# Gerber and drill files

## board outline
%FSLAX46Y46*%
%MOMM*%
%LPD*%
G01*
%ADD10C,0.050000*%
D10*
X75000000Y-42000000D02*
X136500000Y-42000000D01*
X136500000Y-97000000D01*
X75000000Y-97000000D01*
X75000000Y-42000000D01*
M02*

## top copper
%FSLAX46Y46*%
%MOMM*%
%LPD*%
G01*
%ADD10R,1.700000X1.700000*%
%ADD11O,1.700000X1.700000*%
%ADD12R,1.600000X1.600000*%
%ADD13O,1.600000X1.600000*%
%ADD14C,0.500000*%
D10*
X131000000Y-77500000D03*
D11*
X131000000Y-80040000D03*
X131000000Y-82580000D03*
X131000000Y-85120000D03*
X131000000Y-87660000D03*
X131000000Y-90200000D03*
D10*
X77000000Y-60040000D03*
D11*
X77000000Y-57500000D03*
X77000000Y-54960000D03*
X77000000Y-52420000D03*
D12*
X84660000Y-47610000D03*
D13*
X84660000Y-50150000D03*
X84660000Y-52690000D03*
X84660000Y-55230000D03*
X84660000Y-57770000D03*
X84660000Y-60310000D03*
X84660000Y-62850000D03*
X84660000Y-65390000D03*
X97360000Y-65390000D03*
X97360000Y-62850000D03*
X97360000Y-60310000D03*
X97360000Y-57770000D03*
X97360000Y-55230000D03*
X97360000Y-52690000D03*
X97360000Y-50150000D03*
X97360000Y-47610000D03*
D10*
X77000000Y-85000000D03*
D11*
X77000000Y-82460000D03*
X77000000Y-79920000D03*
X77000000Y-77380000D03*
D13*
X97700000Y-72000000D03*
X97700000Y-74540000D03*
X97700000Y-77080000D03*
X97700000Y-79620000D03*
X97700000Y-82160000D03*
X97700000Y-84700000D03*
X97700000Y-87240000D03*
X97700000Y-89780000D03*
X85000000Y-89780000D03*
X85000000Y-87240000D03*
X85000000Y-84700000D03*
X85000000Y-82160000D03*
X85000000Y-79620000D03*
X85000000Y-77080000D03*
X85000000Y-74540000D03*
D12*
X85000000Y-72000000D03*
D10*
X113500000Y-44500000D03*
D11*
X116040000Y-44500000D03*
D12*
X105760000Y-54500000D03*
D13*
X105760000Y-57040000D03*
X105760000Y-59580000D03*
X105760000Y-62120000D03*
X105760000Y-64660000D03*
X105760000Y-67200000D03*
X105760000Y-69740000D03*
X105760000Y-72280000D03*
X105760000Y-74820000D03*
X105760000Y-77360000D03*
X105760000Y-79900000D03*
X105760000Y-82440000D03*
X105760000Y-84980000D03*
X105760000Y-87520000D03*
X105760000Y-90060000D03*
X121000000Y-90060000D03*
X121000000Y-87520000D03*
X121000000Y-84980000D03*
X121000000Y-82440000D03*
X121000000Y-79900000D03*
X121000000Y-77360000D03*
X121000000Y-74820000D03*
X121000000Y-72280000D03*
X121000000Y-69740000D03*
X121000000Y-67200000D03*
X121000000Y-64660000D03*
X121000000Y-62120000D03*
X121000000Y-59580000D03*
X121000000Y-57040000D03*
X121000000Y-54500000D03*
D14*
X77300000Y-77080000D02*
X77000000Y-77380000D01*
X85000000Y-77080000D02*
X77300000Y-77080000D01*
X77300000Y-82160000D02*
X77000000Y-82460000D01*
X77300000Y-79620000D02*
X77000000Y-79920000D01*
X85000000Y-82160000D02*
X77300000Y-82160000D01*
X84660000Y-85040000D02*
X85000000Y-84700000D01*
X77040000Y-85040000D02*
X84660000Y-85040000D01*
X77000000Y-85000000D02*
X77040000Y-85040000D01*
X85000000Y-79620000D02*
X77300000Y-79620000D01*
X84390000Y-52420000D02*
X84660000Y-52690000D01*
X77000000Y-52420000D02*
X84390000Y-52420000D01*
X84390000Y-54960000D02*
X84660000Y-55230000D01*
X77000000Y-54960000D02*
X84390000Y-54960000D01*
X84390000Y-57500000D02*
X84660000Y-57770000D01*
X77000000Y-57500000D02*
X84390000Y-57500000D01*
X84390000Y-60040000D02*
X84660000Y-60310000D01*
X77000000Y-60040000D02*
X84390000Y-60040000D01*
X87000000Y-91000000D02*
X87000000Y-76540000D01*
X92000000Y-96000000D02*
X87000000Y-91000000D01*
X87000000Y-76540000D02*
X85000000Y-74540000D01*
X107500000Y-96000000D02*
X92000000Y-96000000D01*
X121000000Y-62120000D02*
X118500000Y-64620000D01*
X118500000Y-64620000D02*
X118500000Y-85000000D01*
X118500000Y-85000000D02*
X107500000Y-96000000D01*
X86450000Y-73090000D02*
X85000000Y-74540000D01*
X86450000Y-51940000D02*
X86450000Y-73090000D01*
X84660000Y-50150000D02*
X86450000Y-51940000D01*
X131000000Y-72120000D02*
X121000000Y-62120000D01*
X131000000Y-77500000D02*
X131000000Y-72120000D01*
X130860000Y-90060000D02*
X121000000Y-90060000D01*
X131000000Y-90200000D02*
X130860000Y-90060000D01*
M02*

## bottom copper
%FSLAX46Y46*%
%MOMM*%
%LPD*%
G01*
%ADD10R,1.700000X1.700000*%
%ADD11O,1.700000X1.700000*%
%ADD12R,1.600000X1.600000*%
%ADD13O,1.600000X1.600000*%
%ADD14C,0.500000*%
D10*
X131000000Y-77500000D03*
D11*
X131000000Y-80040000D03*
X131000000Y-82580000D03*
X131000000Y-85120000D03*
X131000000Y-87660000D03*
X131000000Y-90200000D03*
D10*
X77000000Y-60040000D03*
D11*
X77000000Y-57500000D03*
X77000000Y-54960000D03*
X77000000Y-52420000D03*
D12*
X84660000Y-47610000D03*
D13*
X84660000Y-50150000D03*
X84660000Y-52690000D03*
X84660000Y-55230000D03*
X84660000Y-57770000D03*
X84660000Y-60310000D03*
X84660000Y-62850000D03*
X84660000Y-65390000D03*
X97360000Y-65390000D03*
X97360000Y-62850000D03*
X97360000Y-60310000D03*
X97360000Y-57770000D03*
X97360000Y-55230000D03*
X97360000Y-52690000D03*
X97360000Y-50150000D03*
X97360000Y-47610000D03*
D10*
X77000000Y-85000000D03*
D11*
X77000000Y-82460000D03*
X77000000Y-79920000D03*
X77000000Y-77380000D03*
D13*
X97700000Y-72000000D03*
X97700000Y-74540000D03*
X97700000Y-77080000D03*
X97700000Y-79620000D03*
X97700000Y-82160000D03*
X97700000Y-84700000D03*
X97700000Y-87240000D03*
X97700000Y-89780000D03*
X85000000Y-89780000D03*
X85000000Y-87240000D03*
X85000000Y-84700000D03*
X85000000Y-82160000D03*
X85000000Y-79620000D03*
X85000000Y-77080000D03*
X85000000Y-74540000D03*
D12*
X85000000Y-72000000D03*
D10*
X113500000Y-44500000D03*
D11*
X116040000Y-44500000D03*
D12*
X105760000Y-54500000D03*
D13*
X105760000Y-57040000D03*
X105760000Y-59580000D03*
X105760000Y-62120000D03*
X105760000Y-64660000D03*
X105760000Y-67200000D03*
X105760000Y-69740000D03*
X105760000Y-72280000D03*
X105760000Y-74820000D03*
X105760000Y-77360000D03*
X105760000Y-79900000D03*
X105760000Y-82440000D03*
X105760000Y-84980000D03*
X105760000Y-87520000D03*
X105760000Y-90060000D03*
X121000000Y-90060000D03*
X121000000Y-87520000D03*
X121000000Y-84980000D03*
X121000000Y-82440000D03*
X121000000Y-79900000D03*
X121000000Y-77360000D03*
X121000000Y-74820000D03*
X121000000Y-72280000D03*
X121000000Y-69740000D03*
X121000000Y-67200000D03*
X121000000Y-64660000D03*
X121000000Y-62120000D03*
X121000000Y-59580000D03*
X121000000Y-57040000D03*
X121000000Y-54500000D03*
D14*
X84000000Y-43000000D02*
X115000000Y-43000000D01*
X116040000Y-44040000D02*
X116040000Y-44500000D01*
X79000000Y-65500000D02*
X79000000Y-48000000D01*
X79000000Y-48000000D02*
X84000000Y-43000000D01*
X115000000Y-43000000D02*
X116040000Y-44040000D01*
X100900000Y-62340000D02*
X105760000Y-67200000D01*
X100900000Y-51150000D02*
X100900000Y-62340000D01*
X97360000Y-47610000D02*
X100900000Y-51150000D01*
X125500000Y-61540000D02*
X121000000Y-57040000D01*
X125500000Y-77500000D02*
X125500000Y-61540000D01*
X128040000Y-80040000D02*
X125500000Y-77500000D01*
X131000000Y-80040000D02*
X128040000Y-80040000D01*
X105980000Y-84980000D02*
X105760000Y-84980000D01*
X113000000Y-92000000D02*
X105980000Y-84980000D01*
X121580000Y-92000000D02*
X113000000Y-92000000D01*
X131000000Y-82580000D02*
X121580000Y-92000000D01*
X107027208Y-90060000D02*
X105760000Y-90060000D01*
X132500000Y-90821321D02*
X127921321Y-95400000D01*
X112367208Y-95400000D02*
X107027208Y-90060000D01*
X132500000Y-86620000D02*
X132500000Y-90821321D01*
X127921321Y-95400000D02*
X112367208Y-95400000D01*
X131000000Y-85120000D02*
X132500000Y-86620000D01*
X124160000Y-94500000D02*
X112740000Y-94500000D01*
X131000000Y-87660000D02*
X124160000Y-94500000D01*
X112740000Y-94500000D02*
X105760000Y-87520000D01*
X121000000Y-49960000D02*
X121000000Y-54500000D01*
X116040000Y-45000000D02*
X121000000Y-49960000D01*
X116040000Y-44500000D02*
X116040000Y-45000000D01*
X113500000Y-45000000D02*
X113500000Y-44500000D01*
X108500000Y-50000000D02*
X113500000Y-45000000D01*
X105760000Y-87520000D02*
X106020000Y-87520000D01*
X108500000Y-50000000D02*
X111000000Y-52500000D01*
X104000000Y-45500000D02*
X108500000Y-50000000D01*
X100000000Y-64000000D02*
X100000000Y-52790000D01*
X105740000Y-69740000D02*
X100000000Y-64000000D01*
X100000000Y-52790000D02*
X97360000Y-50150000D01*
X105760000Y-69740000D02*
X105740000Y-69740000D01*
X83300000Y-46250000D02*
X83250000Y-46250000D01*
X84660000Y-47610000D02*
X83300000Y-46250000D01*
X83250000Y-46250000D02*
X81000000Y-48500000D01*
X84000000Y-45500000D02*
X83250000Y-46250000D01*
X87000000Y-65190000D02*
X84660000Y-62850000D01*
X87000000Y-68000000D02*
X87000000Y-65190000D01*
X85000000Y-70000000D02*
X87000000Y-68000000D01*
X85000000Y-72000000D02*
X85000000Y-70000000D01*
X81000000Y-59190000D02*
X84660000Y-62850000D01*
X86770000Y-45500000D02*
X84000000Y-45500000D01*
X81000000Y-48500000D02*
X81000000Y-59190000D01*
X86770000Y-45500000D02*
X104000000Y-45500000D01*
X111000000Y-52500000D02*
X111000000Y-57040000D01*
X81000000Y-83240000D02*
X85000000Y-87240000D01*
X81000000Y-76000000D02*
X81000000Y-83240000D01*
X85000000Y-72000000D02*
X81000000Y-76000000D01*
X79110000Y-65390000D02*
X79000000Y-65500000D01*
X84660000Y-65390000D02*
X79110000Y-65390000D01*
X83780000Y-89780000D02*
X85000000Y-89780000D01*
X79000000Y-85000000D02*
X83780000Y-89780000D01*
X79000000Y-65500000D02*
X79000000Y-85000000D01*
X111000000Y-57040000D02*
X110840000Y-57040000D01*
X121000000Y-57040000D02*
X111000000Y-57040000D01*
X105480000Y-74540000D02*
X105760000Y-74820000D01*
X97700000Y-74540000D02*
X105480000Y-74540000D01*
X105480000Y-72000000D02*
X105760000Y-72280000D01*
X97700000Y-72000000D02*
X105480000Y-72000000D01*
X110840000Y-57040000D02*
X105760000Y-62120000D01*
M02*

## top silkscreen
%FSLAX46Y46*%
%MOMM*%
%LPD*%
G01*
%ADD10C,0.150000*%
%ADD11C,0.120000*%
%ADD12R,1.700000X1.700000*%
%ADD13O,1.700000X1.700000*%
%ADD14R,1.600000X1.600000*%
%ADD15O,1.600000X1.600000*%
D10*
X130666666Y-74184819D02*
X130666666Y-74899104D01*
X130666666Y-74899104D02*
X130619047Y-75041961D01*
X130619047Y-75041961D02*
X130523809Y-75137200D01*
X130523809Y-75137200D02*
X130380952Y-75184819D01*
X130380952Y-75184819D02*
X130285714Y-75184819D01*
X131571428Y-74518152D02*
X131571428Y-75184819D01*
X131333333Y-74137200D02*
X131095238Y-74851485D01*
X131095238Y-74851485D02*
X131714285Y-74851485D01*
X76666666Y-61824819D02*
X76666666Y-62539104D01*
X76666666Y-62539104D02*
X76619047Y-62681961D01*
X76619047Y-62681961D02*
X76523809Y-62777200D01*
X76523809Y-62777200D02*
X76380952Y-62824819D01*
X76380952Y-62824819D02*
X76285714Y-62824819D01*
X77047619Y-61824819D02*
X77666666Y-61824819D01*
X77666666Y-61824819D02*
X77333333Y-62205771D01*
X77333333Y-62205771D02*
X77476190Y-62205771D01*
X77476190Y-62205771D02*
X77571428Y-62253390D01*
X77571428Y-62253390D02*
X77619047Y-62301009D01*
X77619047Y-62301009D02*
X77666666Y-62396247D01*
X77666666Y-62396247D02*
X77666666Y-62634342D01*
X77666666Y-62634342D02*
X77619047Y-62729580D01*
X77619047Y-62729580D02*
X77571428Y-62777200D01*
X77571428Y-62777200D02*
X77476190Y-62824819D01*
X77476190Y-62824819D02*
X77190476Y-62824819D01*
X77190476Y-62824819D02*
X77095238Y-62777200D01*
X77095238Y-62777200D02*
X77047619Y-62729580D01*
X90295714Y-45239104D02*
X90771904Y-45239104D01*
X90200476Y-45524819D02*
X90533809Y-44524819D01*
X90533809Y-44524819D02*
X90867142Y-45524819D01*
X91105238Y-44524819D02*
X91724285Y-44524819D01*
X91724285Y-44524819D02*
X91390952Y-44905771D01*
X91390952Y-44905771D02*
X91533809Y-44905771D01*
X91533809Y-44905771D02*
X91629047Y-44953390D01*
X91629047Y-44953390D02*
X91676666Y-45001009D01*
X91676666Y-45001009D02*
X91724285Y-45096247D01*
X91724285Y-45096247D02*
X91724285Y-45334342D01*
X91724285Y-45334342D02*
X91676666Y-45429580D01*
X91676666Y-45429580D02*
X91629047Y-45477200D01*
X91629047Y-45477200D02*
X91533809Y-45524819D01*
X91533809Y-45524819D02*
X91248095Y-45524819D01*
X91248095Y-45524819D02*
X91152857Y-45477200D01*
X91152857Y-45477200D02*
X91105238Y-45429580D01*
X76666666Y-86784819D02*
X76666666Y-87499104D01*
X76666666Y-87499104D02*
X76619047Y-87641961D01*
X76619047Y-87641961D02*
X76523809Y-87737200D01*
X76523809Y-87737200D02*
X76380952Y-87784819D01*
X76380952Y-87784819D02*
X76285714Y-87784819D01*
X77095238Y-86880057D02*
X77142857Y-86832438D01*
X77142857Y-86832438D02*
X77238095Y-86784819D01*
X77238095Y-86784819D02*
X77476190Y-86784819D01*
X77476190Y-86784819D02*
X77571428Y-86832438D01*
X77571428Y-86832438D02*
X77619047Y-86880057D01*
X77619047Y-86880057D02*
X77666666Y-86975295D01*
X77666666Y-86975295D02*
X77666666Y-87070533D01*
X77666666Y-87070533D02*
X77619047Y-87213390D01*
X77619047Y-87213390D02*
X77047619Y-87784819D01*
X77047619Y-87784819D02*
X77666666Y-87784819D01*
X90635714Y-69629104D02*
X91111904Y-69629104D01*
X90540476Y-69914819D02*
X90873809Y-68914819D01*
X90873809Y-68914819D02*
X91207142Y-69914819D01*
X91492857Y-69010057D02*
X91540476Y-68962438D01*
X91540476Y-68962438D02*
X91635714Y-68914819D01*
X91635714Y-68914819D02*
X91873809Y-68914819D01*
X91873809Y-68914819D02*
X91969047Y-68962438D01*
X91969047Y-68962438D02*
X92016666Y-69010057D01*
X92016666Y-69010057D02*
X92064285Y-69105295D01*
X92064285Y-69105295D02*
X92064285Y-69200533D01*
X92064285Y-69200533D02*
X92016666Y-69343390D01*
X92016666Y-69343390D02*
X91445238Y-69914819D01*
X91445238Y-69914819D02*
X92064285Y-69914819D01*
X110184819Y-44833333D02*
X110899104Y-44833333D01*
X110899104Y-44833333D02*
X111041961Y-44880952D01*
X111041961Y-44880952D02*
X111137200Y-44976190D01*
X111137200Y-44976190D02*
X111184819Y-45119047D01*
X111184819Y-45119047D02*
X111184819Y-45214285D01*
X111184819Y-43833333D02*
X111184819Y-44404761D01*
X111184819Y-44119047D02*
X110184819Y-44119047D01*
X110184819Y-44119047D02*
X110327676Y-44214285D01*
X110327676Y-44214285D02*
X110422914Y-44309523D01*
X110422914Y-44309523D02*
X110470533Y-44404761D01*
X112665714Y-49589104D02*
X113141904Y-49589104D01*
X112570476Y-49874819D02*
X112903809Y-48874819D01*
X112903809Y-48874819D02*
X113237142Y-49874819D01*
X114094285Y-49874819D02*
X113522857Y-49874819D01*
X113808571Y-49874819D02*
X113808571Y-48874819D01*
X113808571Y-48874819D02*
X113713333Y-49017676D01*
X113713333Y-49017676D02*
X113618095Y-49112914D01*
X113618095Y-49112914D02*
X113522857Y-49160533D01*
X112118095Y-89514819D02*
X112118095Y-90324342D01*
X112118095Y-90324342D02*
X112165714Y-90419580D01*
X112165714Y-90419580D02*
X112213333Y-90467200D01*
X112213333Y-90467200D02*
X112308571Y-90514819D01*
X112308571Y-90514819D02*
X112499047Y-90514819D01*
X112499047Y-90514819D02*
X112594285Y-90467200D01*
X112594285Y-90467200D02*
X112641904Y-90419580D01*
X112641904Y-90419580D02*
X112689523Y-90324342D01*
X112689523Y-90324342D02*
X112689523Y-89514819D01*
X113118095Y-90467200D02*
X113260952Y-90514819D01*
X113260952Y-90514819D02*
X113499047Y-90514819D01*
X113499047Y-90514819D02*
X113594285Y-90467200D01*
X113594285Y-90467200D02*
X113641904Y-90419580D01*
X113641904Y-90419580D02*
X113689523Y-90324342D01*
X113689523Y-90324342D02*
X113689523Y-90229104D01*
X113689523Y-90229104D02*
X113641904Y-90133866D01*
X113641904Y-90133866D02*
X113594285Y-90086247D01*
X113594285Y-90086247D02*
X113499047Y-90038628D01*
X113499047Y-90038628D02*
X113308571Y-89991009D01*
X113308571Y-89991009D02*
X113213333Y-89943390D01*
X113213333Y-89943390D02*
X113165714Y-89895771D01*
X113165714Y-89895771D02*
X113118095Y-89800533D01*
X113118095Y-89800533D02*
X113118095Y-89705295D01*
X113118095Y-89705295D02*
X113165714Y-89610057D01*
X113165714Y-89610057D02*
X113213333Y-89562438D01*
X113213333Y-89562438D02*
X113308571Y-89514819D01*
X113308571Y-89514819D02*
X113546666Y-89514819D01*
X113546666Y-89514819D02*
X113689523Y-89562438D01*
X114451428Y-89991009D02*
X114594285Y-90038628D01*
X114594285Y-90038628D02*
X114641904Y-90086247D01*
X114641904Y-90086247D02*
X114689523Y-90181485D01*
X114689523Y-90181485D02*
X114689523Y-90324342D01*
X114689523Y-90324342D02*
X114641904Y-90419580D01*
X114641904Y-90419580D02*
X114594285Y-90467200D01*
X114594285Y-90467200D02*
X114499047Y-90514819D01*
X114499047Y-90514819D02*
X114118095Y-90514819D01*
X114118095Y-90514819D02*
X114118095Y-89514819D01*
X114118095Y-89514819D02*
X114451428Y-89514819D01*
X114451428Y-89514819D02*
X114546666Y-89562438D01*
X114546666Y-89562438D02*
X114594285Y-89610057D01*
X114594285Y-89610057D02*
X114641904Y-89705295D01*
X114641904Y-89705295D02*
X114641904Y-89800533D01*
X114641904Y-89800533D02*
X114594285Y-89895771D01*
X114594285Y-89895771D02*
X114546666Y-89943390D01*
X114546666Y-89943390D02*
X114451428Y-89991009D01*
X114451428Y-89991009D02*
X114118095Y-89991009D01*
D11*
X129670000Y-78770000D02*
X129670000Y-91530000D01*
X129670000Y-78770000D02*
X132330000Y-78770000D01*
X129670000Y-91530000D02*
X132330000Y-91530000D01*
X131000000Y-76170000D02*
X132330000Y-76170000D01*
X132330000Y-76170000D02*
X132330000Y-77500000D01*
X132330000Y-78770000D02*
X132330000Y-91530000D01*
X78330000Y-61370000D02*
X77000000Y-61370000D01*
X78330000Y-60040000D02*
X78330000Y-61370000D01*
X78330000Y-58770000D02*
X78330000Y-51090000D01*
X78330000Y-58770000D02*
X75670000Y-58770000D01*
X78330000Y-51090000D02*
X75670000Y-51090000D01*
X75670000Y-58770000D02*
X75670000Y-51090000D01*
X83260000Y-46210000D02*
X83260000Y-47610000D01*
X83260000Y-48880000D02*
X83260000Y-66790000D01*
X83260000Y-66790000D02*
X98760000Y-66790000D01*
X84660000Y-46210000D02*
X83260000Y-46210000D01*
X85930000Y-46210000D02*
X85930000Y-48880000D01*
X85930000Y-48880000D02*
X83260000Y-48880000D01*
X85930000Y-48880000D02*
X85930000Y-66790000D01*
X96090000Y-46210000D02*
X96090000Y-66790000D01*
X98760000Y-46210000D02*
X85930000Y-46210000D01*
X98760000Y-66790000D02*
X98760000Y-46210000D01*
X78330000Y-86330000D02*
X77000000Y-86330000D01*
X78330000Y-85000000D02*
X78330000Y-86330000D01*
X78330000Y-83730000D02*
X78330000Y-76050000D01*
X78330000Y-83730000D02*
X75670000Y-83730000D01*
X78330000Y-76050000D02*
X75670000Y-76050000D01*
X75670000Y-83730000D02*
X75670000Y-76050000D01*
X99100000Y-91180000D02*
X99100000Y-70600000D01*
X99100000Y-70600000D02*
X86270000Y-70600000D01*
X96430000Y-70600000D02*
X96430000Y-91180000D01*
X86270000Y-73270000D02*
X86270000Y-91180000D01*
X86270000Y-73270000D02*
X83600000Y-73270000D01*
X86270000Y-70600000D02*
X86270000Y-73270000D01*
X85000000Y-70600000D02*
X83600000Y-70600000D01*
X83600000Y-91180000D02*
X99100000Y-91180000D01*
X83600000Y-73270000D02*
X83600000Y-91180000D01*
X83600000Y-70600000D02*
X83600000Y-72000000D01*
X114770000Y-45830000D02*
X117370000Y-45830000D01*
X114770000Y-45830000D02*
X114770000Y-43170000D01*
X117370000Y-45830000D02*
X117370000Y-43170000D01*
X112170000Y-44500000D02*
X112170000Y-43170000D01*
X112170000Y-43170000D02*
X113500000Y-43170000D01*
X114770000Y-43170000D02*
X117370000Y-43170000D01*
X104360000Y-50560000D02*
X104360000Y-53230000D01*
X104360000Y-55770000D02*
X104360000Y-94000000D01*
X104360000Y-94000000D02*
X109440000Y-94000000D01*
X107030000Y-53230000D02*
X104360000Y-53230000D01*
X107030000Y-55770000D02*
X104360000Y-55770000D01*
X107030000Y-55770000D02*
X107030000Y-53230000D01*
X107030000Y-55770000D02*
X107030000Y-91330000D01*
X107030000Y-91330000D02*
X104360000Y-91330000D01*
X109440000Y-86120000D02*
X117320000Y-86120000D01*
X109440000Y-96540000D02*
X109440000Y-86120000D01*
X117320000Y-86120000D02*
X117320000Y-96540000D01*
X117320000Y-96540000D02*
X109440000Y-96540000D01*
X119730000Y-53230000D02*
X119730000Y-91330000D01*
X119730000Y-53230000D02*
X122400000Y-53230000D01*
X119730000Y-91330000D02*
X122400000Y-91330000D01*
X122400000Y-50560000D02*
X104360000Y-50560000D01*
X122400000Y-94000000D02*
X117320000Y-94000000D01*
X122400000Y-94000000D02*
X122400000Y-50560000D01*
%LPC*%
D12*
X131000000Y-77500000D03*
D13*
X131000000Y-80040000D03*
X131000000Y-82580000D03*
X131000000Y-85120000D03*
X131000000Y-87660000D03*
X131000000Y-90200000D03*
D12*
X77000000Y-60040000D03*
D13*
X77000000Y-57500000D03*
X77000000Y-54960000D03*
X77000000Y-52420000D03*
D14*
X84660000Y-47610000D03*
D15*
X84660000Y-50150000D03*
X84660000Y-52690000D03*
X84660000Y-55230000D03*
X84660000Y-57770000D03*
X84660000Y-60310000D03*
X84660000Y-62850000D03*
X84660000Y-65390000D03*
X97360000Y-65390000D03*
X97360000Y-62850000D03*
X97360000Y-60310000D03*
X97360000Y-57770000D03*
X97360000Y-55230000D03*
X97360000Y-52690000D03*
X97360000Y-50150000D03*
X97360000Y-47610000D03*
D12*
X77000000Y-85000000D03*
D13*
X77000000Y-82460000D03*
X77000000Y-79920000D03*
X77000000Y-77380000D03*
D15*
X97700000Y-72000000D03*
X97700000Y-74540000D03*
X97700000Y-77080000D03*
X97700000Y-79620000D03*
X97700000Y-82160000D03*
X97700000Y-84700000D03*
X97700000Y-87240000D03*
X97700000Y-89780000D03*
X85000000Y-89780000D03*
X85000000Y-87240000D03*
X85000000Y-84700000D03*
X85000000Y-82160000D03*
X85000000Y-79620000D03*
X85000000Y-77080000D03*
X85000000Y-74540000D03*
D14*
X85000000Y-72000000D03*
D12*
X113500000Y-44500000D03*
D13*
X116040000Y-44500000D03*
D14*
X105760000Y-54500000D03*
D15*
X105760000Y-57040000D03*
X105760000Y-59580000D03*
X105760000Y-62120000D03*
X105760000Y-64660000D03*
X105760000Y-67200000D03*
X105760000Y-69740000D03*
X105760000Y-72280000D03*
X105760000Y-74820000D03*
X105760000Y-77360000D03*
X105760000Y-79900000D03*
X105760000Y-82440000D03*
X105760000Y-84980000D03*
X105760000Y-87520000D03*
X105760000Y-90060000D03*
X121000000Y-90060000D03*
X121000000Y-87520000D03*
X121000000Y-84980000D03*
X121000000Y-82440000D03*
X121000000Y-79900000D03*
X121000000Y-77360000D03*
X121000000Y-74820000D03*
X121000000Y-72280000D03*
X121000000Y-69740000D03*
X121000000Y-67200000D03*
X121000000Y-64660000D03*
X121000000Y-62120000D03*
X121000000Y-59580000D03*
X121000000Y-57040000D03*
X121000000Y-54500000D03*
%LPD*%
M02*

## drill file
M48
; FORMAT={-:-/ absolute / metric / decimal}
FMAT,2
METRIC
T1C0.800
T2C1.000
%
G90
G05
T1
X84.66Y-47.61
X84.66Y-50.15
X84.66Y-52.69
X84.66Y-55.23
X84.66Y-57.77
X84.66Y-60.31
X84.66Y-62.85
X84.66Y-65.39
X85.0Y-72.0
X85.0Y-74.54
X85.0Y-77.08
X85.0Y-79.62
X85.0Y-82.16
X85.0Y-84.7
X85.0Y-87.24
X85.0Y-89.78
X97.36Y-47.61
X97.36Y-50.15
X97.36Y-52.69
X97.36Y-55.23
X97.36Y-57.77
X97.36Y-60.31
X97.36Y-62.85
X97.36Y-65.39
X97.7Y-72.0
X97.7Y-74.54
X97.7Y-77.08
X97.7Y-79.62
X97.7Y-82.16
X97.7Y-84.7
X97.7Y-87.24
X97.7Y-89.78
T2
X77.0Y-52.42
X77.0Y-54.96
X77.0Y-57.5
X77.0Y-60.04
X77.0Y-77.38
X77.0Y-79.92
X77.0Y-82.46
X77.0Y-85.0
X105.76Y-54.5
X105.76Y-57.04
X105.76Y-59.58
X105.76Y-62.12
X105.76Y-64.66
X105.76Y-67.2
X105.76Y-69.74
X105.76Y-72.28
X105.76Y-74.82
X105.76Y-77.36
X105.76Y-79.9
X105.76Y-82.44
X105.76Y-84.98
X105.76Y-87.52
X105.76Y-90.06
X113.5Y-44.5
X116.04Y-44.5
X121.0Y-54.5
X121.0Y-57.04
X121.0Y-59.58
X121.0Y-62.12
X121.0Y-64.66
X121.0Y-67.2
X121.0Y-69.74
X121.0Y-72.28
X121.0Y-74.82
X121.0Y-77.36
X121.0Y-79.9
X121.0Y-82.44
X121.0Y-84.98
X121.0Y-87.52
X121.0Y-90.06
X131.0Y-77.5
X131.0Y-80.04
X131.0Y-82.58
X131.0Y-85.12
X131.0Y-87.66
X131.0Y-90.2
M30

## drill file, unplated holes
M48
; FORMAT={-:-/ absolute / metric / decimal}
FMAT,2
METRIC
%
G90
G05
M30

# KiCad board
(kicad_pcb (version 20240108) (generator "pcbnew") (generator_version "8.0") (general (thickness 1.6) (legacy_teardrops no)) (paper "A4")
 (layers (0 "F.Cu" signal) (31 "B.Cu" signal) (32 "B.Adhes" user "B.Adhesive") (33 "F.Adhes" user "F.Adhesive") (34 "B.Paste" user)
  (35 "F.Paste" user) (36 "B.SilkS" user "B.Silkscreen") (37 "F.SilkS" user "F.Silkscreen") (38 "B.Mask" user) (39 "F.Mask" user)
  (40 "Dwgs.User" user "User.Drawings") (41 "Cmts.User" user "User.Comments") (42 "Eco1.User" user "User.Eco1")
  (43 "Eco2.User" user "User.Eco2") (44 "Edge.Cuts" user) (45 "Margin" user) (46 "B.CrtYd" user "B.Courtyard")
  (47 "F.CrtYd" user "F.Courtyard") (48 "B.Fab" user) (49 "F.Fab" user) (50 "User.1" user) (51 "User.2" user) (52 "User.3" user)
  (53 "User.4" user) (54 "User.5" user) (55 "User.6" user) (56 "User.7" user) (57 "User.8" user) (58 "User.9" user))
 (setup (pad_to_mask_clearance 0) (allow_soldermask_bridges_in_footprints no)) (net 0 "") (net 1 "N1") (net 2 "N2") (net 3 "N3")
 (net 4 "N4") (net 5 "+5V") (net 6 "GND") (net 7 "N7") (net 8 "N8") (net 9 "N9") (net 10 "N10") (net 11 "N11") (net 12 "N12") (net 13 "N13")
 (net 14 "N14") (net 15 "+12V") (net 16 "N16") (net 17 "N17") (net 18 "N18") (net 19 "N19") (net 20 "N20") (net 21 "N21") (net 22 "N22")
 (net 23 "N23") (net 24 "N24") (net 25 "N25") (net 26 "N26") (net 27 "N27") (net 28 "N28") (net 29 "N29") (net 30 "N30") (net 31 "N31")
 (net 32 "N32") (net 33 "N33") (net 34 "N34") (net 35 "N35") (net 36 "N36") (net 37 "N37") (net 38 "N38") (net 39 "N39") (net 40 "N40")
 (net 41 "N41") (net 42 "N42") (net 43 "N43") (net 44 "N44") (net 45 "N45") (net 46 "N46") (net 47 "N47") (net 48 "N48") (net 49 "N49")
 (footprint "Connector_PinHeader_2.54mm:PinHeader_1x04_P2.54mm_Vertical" (layer "F.Cu") (at 77 85 180)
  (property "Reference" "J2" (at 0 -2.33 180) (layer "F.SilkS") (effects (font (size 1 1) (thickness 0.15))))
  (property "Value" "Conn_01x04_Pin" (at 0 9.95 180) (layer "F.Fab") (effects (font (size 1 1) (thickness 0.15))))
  (fp_line (start 1.33 1.27) (end 1.33 8.95) (stroke (width 0.12) (type solid)) (layer "F.SilkS"))
  (fp_line (start -1.33 8.95) (end 1.33 8.95) (stroke (width 0.12) (type solid)) (layer "F.SilkS"))
  (fp_line (start -1.33 1.27) (end 1.33 1.27) (stroke (width 0.12) (type solid)) (layer "F.SilkS"))
  (fp_line (start -1.33 1.27) (end -1.33 8.95) (stroke (width 0.12) (type solid)) (layer "F.SilkS"))
  (fp_line (start -1.33 0) (end -1.33 -1.33) (stroke (width 0.12) (type solid)) (layer "F.SilkS"))
  (fp_line (start -1.33 -1.33) (end 0 -1.33) (stroke (width 0.12) (type solid)) (layer "F.SilkS"))
  (pad "1" thru_hole rect (at 0 0 180) (size 1.7 1.7) (drill 1) (layers "*.Cu" "*.Mask") (remove_unused_layers no) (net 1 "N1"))
  (pad "2" thru_hole oval (at 0 2.54 180) (size 1.7 1.7) (drill 1) (layers "*.Cu" "*.Mask") (remove_unused_layers no) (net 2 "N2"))
  (pad "3" thru_hole oval (at 0 5.08 180) (size 1.7 1.7) (drill 1) (layers "*.Cu" "*.Mask") (remove_unused_layers no) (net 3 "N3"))
  (pad "4" thru_hole oval (at 0 7.62 180) (size 1.7 1.7) (drill 1) (layers "*.Cu" "*.Mask") (remove_unused_layers no) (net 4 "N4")))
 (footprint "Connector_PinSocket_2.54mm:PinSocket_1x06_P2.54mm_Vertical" (layer "F.Cu") (at 131 77.5)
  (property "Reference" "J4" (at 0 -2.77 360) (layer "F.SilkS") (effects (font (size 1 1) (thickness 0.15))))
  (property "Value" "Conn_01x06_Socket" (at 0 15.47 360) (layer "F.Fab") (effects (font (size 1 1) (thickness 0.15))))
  (fp_line (start -1.33 1.27) (end -1.33 14.03) (stroke (width 0.12) (type solid)) (layer "F.SilkS"))
  (fp_line (start -1.33 1.27) (end 1.33 1.27) (stroke (width 0.12) (type solid)) (layer "F.SilkS"))
  (fp_line (start -1.33 14.03) (end 1.33 14.03) (stroke (width 0.12) (type solid)) (layer "F.SilkS"))
  (fp_line (start 0 -1.33) (end 1.33 -1.33) (stroke (width 0.12) (type solid)) (layer "F.SilkS"))
  (fp_line (start 1.33 -1.33) (end 1.33 0) (stroke (width 0.12) (type solid)) (layer "F.SilkS"))
  (fp_line (start 1.33 1.27) (end 1.33 14.03) (stroke (width 0.12) (type solid)) (layer "F.SilkS"))
  (pad "1" thru_hole rect (at 0 0) (size 1.7 1.7) (drill 1) (layers "*.Cu" "*.Mask") (remove_unused_layers no) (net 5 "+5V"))
  (pad "2" thru_hole oval (at 0 2.54) (size 1.7 1.7) (drill 1) (layers "*.Cu" "*.Mask") (remove_unused_layers no) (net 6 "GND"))
  (pad "3" thru_hole oval (at 0 5.08) (size 1.7 1.7) (drill 1) (layers "*.Cu" "*.Mask") (remove_unused_layers no) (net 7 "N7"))
  (pad "4" thru_hole oval (at 0 7.62) (size 1.7 1.7) (drill 1) (layers "*.Cu" "*.Mask") (remove_unused_layers no) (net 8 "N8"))
  (pad "5" thru_hole oval (at 0 10.16) (size 1.7 1.7) (drill 1) (layers "*.Cu" "*.Mask") (remove_unused_layers no) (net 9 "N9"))
  (pad "6" thru_hole oval (at 0 12.7) (size 1.7 1.7) (drill 1) (layers "*.Cu" "*.Mask") (remove_unused_layers no) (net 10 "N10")))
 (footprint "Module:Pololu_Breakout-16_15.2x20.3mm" (layer "F.Cu") (at 84.66 47.61)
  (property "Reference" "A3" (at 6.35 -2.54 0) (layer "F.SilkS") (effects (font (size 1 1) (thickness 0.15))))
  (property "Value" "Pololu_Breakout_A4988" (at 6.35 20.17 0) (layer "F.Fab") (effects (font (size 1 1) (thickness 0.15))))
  (fp_line (start -1.4 -1.4) (end -1.4 0) (stroke (width 0.12) (type solid)) (layer "F.SilkS"))
  (fp_line (start -1.4 1.27) (end -1.4 19.18) (stroke (width 0.12) (type solid)) (layer "F.SilkS"))
  (fp_line (start -1.4 19.18) (end 14.1 19.18) (stroke (width 0.12) (type solid)) (layer "F.SilkS"))
  (fp_line (start 0 -1.4) (end -1.4 -1.4) (stroke (width 0.12) (type solid)) (layer "F.SilkS"))
  (fp_line (start 1.27 -1.4) (end 1.27 1.27) (stroke (width 0.12) (type solid)) (layer "F.SilkS"))
  (fp_line (start 1.27 1.27) (end -1.4 1.27) (stroke (width 0.12) (type solid)) (layer "F.SilkS"))
  (fp_line (start 1.27 1.27) (end 1.27 19.18) (stroke (width 0.12) (type solid)) (layer "F.SilkS"))
  (fp_line (start 11.43 -1.4) (end 11.43 19.18) (stroke (width 0.12) (type solid)) (layer "F.SilkS"))
  (fp_line (start 14.1 -1.4) (end 1.27 -1.4) (stroke (width 0.12) (type solid)) (layer "F.SilkS"))
  (fp_line (start 14.1 19.18) (end 14.1 -1.4) (stroke (width 0.12) (type solid)) (layer "F.SilkS"))
  (pad "1" thru_hole rect (at 0 0) (size 1.6 1.6) (drill 0.8) (layers "*.Cu" "*.Mask") (remove_unused_layers no) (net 6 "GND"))
  (pad "2" thru_hole oval (at 0 2.54) (size 1.6 1.6) (drill 0.8) (layers "*.Cu" "*.Mask") (remove_unused_layers no) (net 5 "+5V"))
  (pad "3" thru_hole oval (at 0 5.08) (size 1.6 1.6) (drill 0.8) (layers "*.Cu" "*.Mask") (remove_unused_layers no) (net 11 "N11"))
  (pad "4" thru_hole oval (at 0 7.62) (size 1.6 1.6) (drill 0.8) (layers "*.Cu" "*.Mask") (remove_unused_layers no) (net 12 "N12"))
  (pad "5" thru_hole oval (at 0 10.16) (size 1.6 1.6) (drill 0.8) (layers "*.Cu" "*.Mask") (remove_unused_layers no) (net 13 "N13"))
  (pad "6" thru_hole oval (at 0 12.7) (size 1.6 1.6) (drill 0.8) (layers "*.Cu" "*.Mask") (remove_unused_layers no) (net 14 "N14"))
  (pad "7" thru_hole oval (at 0 15.24) (size 1.6 1.6) (drill 0.8) (layers "*.Cu" "*.Mask") (remove_unused_layers no) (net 6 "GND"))
  (pad "8" thru_hole oval (at 0 17.78) (size 1.6 1.6) (drill 0.8) (layers "*.Cu" "*.Mask") (remove_unused_layers no) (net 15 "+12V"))
  (pad "9" thru_hole oval (at 12.7 17.78) (size 1.6 1.6) (drill 0.8) (layers "*.Cu" "*.Mask") (remove_unused_layers no) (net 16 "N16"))
  (pad "10" thru_hole oval (at 12.7 15.24) (size 1.6 1.6) (drill 0.8) (layers "*.Cu" "*.Mask") (remove_unused_layers no) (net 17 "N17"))
  (pad "11" thru_hole oval (at 12.7 12.7) (size 1.6 1.6) (drill 0.8) (layers "*.Cu" "*.Mask") (remove_unused_layers no) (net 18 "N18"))
  (pad "12" thru_hole oval (at 12.7 10.16) (size 1.6 1.6) (drill 0.8) (layers "*.Cu" "*.Mask") (remove_unused_layers no) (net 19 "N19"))
  (pad "13" thru_hole oval (at 12.7 7.62) (size 1.6 1.6) (drill 0.8) (layers "*.Cu" "*.Mask") (remove_unused_layers no) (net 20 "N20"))
  (pad "14" thru_hole oval (at 12.7 5.08) (size 1.6 1.6) (drill 0.8) (layers "*.Cu" "*.Mask") (remove_unused_layers no) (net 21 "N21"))
  (pad "15" thru_hole oval (at 12.7 2.54) (size 1.6 1.6) (drill 0.8) (layers "*.Cu" "*.Mask") (remove_unused_layers no) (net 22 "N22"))
  (pad "16" thru_hole oval (at 12.7 0) (size 1.6 1.6) (drill 0.8) (layers "*.Cu" "*.Mask") (remove_unused_layers no) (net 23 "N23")))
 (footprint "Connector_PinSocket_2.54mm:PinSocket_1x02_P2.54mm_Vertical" (layer "F.Cu") (at 113.5 44.5 90)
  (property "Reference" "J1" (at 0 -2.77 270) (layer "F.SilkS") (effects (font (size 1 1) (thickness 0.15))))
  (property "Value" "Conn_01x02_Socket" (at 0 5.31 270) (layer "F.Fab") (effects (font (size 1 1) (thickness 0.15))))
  (fp_line (start 1.33 -1.33) (end 1.33 0) (stroke (width 0.12) (type solid)) (layer "F.SilkS"))
  (fp_line (start 0 -1.33) (end 1.33 -1.33) (stroke (width 0.12) (type solid)) (layer "F.SilkS"))
  (fp_line (start 1.33 1.27) (end 1.33 3.87) (stroke (width 0.12) (type solid)) (layer "F.SilkS"))
  (fp_line (start -1.33 1.27) (end 1.33 1.27) (stroke (width 0.12) (type solid)) (layer "F.SilkS"))
  (fp_line (start -1.33 1.27) (end -1.33 3.87) (stroke (width 0.12) (type solid)) (layer "F.SilkS"))
  (fp_line (start -1.33 3.87) (end 1.33 3.87) (stroke (width 0.12) (type solid)) (layer "F.SilkS"))
  (pad "1" thru_hole rect (at 0 0 90) (size 1.7 1.7) (drill 1) (layers "*.Cu" "*.Mask") (remove_unused_layers no) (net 6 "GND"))
  (pad "2" thru_hole oval (at 0 2.54 90) (size 1.7 1.7) (drill 1) (layers "*.Cu" "*.Mask") (remove_unused_layers no) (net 15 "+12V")))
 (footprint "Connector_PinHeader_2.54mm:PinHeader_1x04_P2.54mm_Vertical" (layer "F.Cu") (at 77 60.04 180)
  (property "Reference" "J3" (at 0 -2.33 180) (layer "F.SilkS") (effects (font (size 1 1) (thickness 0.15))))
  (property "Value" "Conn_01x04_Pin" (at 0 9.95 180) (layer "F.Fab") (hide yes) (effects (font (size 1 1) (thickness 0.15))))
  (fp_line (start 1.33 1.27) (end 1.33 8.95) (stroke (width 0.12) (type solid)) (layer "F.SilkS"))
  (fp_line (start -1.33 8.95) (end 1.33 8.95) (stroke (width 0.12) (type solid)) (layer "F.SilkS"))
  (fp_line (start -1.33 1.27) (end 1.33 1.27) (stroke (width 0.12) (type solid)) (layer "F.SilkS"))
  (fp_line (start -1.33 1.27) (end -1.33 8.95) (stroke (width 0.12) (type solid)) (layer "F.SilkS"))
  (fp_line (start -1.33 0) (end -1.33 -1.33) (stroke (width 0.12) (type solid)) (layer "F.SilkS"))
  (fp_line (start -1.33 -1.33) (end 0 -1.33) (stroke (width 0.12) (type solid)) (layer "F.SilkS"))
  (pad "1" thru_hole rect (at 0 0 180) (size 1.7 1.7) (drill 1) (layers "*.Cu" "*.Mask") (remove_unused_layers no) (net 14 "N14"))
  (pad "2" thru_hole oval (at 0 2.54 180) (size 1.7 1.7) (drill 1) (layers "*.Cu" "*.Mask") (remove_unused_layers no) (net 13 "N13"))
  (pad "3" thru_hole oval (at 0 5.08 180) (size 1.7 1.7) (drill 1) (layers "*.Cu" "*.Mask") (remove_unused_layers no) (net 12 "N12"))
  (pad "4" thru_hole oval (at 0 7.62 180) (size 1.7 1.7) (drill 1) (layers "*.Cu" "*.Mask") (remove_unused_layers no) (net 11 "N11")))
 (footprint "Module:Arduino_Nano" (layer "F.Cu") (at 105.76 54.5)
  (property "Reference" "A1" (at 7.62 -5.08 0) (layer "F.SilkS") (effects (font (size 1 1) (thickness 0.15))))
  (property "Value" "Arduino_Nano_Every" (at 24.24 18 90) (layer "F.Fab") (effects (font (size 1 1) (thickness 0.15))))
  (fp_line (start -1.4 -3.94) (end -1.4 -1.27) (stroke (width 0.12) (type solid)) (layer "F.SilkS"))
  (fp_line (start -1.4 1.27) (end -1.4 39.5) (stroke (width 0.12) (type solid)) (layer "F.SilkS"))
  (fp_line (start -1.4 39.5) (end 3.68 39.5) (stroke (width 0.12) (type solid)) (layer "F.SilkS"))
  (fp_line (start 1.27 -1.27) (end -1.4 -1.27) (stroke (width 0.12) (type solid)) (layer "F.SilkS"))
  (fp_line (start 1.27 1.27) (end -1.4 1.27) (stroke (width 0.12) (type solid)) (layer "F.SilkS"))
  (fp_line (start 1.27 1.27) (end 1.27 -1.27) (stroke (width 0.12) (type solid)) (layer "F.SilkS"))
  (fp_line (start 1.27 1.27) (end 1.27 36.83) (stroke (width 0.12) (type solid)) (layer "F.SilkS"))
  (fp_line (start 1.27 36.83) (end -1.4 36.83) (stroke (width 0.12) (type solid)) (layer "F.SilkS"))
  (fp_line (start 3.68 31.62) (end 11.56 31.62) (stroke (width 0.12) (type solid)) (layer "F.SilkS"))
  (fp_line (start 3.68 42.04) (end 3.68 31.62) (stroke (width 0.12) (type solid)) (layer "F.SilkS"))
  (fp_line (start 11.56 31.62) (end 11.56 42.04) (stroke (width 0.12) (type solid)) (layer "F.SilkS"))
  (fp_line (start 11.56 42.04) (end 3.68 42.04) (stroke (width 0.12) (type solid)) (layer "F.SilkS"))
  (fp_line (start 13.97 -1.27) (end 13.97 36.83) (stroke (width 0.12) (type solid)) (layer "F.SilkS"))
  (fp_line (start 13.97 -1.27) (end 16.64 -1.27) (stroke (width 0.12) (type solid)) (layer "F.SilkS"))
  (fp_line (start 13.97 36.83) (end 16.64 36.83) (stroke (width 0.12) (type solid)) (layer "F.SilkS"))
  (fp_line (start 16.64 -3.94) (end -1.4 -3.94) (stroke (width 0.12) (type solid)) (layer "F.SilkS"))
  (fp_line (start 16.64 39.5) (end 11.56 39.5) (stroke (width 0.12) (type solid)) (layer "F.SilkS"))
  (fp_line (start 16.64 39.5) (end 16.64 -3.94) (stroke (width 0.12) (type solid)) (layer "F.SilkS"))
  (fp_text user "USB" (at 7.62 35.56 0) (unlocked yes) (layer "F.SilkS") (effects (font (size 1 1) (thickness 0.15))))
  (pad "1" thru_hole rect (at 0 0) (size 1.6 1.6) (drill 1) (layers "*.Cu" "*.Mask") (remove_unused_layers no) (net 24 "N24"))
  (pad "2" thru_hole oval (at 0 2.54) (size 1.6 1.6) (drill 1) (layers "*.Cu" "*.Mask") (remove_unused_layers no) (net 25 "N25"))
  (pad "3" thru_hole oval (at 0 5.08) (size 1.6 1.6) (drill 1) (layers "*.Cu" "*.Mask") (remove_unused_layers no) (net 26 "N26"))
  (pad "4" thru_hole oval (at 0 7.62) (size 1.6 1.6) (drill 1) (layers "*.Cu" "*.Mask") (remove_unused_layers no) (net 6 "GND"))
  (pad "5" thru_hole oval (at 0 10.16) (size 1.6 1.6) (drill 1) (layers "*.Cu" "*.Mask") (remove_unused_layers no) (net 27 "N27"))
  (pad "6" thru_hole oval (at 0 12.7) (size 1.6 1.6) (drill 1) (layers "*.Cu" "*.Mask") (remove_unused_layers no) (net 23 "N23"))
  (pad "7" thru_hole oval (at 0 15.24) (size 1.6 1.6) (drill 1) (layers "*.Cu" "*.Mask") (remove_unused_layers no) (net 22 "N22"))
  (pad "8" thru_hole oval (at 0 17.78) (size 1.6 1.6) (drill 1) (layers "*.Cu" "*.Mask") (remove_unused_layers no) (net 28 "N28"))
  (pad "9" thru_hole oval (at 0 20.32) (size 1.6 1.6) (drill 1) (layers "*.Cu" "*.Mask") (remove_unused_layers no) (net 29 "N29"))
  (pad "10" thru_hole oval (at 0 22.86) (size 1.6 1.6) (drill 1) (layers "*.Cu" "*.Mask") (remove_unused_layers no) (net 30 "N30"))
  (pad "11" thru_hole oval (at 0 25.4) (size 1.6 1.6) (drill 1) (layers "*.Cu" "*.Mask") (remove_unused_layers no) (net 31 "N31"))
  (pad "12" thru_hole oval (at 0 27.94) (size 1.6 1.6) (drill 1) (layers "*.Cu" "*.Mask") (remove_unused_layers no) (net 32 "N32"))
  (pad "13" thru_hole oval (at 0 30.48) (size 1.6 1.6) (drill 1) (layers "*.Cu" "*.Mask") (remove_unused_layers no) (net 7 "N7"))
  (pad "14" thru_hole oval (at 0 33.02) (size 1.6 1.6) (drill 1) (layers "*.Cu" "*.Mask") (remove_unused_layers no) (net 9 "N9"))
  (pad "15" thru_hole oval (at 0 35.56) (size 1.6 1.6) (drill 1) (layers "*.Cu" "*.Mask") (remove_unused_layers no) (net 8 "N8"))
  (pad "16" thru_hole oval (at 15.24 35.56) (size 1.6 1.6) (drill 1) (layers "*.Cu" "*.Mask") (remove_unused_layers no) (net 10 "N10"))
  (pad "17" thru_hole oval (at 15.24 33.02) (size 1.6 1.6) (drill 1) (layers "*.Cu" "*.Mask") (remove_unused_layers no) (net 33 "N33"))
  (pad "18" thru_hole oval (at 15.24 30.48) (size 1.6 1.6) (drill 1) (layers "*.Cu" "*.Mask") (remove_unused_layers no) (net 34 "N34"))
  (pad "19" thru_hole oval (at 15.24 27.94) (size 1.6 1.6) (drill 1) (layers "*.Cu" "*.Mask") (remove_unused_layers no) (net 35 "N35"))
  (pad "20" thru_hole oval (at 15.24 25.4) (size 1.6 1.6) (drill 1) (layers "*.Cu" "*.Mask") (remove_unused_layers no) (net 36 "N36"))
  (pad "21" thru_hole oval (at 15.24 22.86) (size 1.6 1.6) (drill 1) (layers "*.Cu" "*.Mask") (remove_unused_layers no) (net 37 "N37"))
  (pad "22" thru_hole oval (at 15.24 20.32) (size 1.6 1.6) (drill 1) (layers "*.Cu" "*.Mask") (remove_unused_layers no) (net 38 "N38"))
  (pad "23" thru_hole oval (at 15.24 17.78) (size 1.6 1.6) (drill 1) (layers "*.Cu" "*.Mask") (remove_unused_layers no) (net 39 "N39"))
  (pad "24" thru_hole oval (at 15.24 15.24) (size 1.6 1.6) (drill 1) (layers "*.Cu" "*.Mask") (remove_unused_layers no) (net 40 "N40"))
  (pad "25" thru_hole oval (at 15.24 12.7) (size 1.6 1.6) (drill 1) (layers "*.Cu" "*.Mask") (remove_unused_layers no) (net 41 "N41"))
  (pad "26" thru_hole oval (at 15.24 10.16) (size 1.6 1.6) (drill 1) (layers "*.Cu" "*.Mask") (remove_unused_layers no) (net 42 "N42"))
  (pad "27" thru_hole oval (at 15.24 7.62) (size 1.6 1.6) (drill 1) (layers "*.Cu" "*.Mask") (remove_unused_layers no) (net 5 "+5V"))
  (pad "28" thru_hole oval (at 15.24 5.08) (size 1.6 1.6) (drill 1) (layers "*.Cu" "*.Mask") (remove_unused_layers no) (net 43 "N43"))
  (pad "29" thru_hole oval (at 15.24 2.54) (size 1.6 1.6) (drill 1) (layers "*.Cu" "*.Mask") (remove_unused_layers no) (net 6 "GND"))
  (pad "30" thru_hole oval (at 15.24 0) (size 1.6 1.6) (drill 1) (layers "*.Cu" "*.Mask") (remove_unused_layers no) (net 15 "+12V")))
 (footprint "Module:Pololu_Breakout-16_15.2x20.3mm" (layer "F.Cu") (at 85 72)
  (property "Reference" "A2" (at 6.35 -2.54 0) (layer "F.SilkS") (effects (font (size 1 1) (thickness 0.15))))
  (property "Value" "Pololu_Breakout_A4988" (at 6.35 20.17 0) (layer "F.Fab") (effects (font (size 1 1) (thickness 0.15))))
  (fp_line (start -1.4 -1.4) (end -1.4 0) (stroke (width 0.12) (type solid)) (layer "F.SilkS"))
  (fp_line (start -1.4 1.27) (end -1.4 19.18) (stroke (width 0.12) (type solid)) (layer "F.SilkS"))
  (fp_line (start -1.4 19.18) (end 14.1 19.18) (stroke (width 0.12) (type solid)) (layer "F.SilkS"))
  (fp_line (start 0 -1.4) (end -1.4 -1.4) (stroke (width 0.12) (type solid)) (layer "F.SilkS"))
  (fp_line (start 1.27 -1.4) (end 1.27 1.27) (stroke (width 0.12) (type solid)) (layer "F.SilkS"))
  (fp_line (start 1.27 1.27) (end -1.4 1.27) (stroke (width 0.12) (type solid)) (layer "F.SilkS"))
  (fp_line (start 1.27 1.27) (end 1.27 19.18) (stroke (width 0.12) (type solid)) (layer "F.SilkS"))
  (fp_line (start 11.43 -1.4) (end 11.43 19.18) (stroke (width 0.12) (type solid)) (layer "F.SilkS"))
  (fp_line (start 14.1 -1.4) (end 1.27 -1.4) (stroke (width 0.12) (type solid)) (layer "F.SilkS"))
  (fp_line (start 14.1 19.18) (end 14.1 -1.4) (stroke (width 0.12) (type solid)) (layer "F.SilkS"))
  (pad "1" thru_hole rect (at 0 0) (size 1.6 1.6) (drill 0.8) (layers "*.Cu" "*.Mask") (remove_unused_layers no) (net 6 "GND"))
  (pad "2" thru_hole oval (at 0 2.54) (size 1.6 1.6) (drill 0.8) (layers "*.Cu" "*.Mask") (remove_unused_layers no) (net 5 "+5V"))
  (pad "3" thru_hole oval (at 0 5.08) (size 1.6 1.6) (drill 0.8) (layers "*.Cu" "*.Mask") (remove_unused_layers no) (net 4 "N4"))
  (pad "4" thru_hole oval (at 0 7.62) (size 1.6 1.6) (drill 0.8) (layers "*.Cu" "*.Mask") (remove_unused_layers no) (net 3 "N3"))
  (pad "5" thru_hole oval (at 0 10.16) (size 1.6 1.6) (drill 0.8) (layers "*.Cu" "*.Mask") (remove_unused_layers no) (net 2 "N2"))
  (pad "6" thru_hole oval (at 0 12.7) (size 1.6 1.6) (drill 0.8) (layers "*.Cu" "*.Mask") (remove_unused_layers no) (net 1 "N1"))
  (pad "7" thru_hole oval (at 0 15.24) (size 1.6 1.6) (drill 0.8) (layers "*.Cu" "*.Mask") (remove_unused_layers no) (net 6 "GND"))
  (pad "8" thru_hole oval (at 0 17.78) (size 1.6 1.6) (drill 0.8) (layers "*.Cu" "*.Mask") (remove_unused_layers no) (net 15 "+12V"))
  (pad "9" thru_hole oval (at 12.7 17.78) (size 1.6 1.6) (drill 0.8) (layers "*.Cu" "*.Mask") (remove_unused_layers no) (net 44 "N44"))
  (pad "10" thru_hole oval (at 12.7 15.24) (size 1.6 1.6) (drill 0.8) (layers "*.Cu" "*.Mask") (remove_unused_layers no) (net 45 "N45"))
  (pad "11" thru_hole oval (at 12.7 12.7) (size 1.6 1.6) (drill 0.8) (layers "*.Cu" "*.Mask") (remove_unused_layers no) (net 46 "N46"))
  (pad "12" thru_hole oval (at 12.7 10.16) (size 1.6 1.6) (drill 0.8) (layers "*.Cu" "*.Mask") (remove_unused_layers no) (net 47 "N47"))
  (pad "13" thru_hole oval (at 12.7 7.62) (size 1.6 1.6) (drill 0.8) (layers "*.Cu" "*.Mask") (remove_unused_layers no) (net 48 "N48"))
  (pad "14" thru_hole oval (at 12.7 5.08) (size 1.6 1.6) (drill 0.8) (layers "*.Cu" "*.Mask") (remove_unused_layers no) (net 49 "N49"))
  (pad "15" thru_hole oval (at 12.7 2.54) (size 1.6 1.6) (drill 0.8) (layers "*.Cu" "*.Mask") (remove_unused_layers no) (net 29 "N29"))
  (pad "16" thru_hole oval (at 12.7 0) (size 1.6 1.6) (drill 0.8) (layers "*.Cu" "*.Mask") (remove_unused_layers no) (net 28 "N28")))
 (gr_rect (start 75 42) (end 136.5 97) (stroke (width 0.05) (type default)) (fill none) (layer "Edge.Cuts"))
 (segment (start 83.25 46.25) (end 81 48.5) (width 0.5) (layer "B.Cu") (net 6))
 (segment (start 81 76) (end 81 83.24) (width 0.5) (layer "B.Cu") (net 6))
 (segment (start 87 68) (end 87 65.19) (width 0.5) (layer "B.Cu") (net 6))
 (segment (start 104 45.5) (end 108.5 50) (width 0.5) (layer "B.Cu") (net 6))
 (segment (start 131 80.04) (end 128.04 80.04) (width 0.5) (layer "B.Cu") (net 6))
 (segment (start 81 48.5) (end 81 59.19) (width 0.5) (layer "B.Cu") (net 6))
 (segment (start 85 72) (end 85 70) (width 0.5) (layer "B.Cu") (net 6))
 (segment (start 86.77 45.5) (end 84 45.5) (width 0.5) (layer "B.Cu") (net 6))
 (segment (start 81 83.24) (end 85 87.24) (width 0.5) (layer "B.Cu") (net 6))
 (segment (start 125.5 77.5) (end 125.5 61.54) (width 0.5) (layer "B.Cu") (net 6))
 (segment (start 121 57.04) (end 111 57.04) (width 0.5) (layer "B.Cu") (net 6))
 (segment (start 128.04 80.04) (end 125.5 77.5) (width 0.5) (layer "B.Cu") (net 6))
 (segment (start 87 65.19) (end 84.66 62.85) (width 0.5) (layer "B.Cu") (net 6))
 (segment (start 83.3 46.25) (end 83.25 46.25) (width 0.5) (layer "B.Cu") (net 6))
 (segment (start 108.5 50) (end 111 52.5) (width 0.5) (layer "B.Cu") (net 6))
 (segment (start 84.66 47.61) (end 83.3 46.25) (width 0.5) (layer "B.Cu") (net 6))
 (segment (start 84 45.5) (end 83.25 46.25) (width 0.5) (layer "B.Cu") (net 6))
 (segment (start 111 57.04) (end 110.84 57.04) (width 0.5) (layer "B.Cu") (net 6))
 (segment (start 125.5 61.54) (end 121 57.04) (width 0.5) (layer "B.Cu") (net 6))
 (segment (start 110.84 57.04) (end 105.76 62.12) (width 0.5) (layer "B.Cu") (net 6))
 (segment (start 111 52.5) (end 111 57.04) (width 0.5) (layer "B.Cu") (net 6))
 (segment (start 108.5 50) (end 113.5 45) (width 0.5) (layer "B.Cu") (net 6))
 (segment (start 85 72) (end 81 76) (width 0.5) (layer "B.Cu") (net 6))
 (segment (start 113.5 45) (end 113.5 44.5) (width 0.5) (layer "B.Cu") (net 6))
 (segment (start 86.77 45.5) (end 104 45.5) (width 0.5) (layer "B.Cu") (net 6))
 (segment (start 81 59.19) (end 84.66 62.85) (width 0.5) (layer "B.Cu") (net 6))
 (segment (start 85 70) (end 87 68) (width 0.5) (layer "B.Cu") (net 6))
 (segment (start 79 48) (end 84 43) (width 0.5) (layer "B.Cu") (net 15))
 (segment (start 79.11 65.39) (end 79 65.5) (width 0.5) (layer "B.Cu") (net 15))
 (segment (start 115 43) (end 116.04 44.04) (width 0.5) (layer "B.Cu") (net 15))
 (segment (start 79 65.5) (end 79 85) (width 0.5) (layer "B.Cu") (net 15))
 (segment (start 116.04 44.5) (end 116.04 45) (width 0.5) (layer "B.Cu") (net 15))
 (segment (start 83.78 89.78) (end 85 89.78) (width 0.5) (layer "B.Cu") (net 15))
 (segment (start 116.04 44.04) (end 116.04 44.5) (width 0.5) (layer "B.Cu") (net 15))
 (segment (start 121 49.96) (end 121 54.5) (width 0.5) (layer "B.Cu") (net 15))
 (segment (start 84 43) (end 115 43) (width 0.5) (layer "B.Cu") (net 15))
 (segment (start 84.66 65.39) (end 79.11 65.39) (width 0.5) (layer "B.Cu") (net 15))
 (segment (start 116.04 45) (end 121 49.96) (width 0.5) (layer "B.Cu") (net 15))
 (segment (start 79 85) (end 83.78 89.78) (width 0.5) (layer "B.Cu") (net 15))
 (segment (start 79 65.5) (end 79 48) (width 0.5) (layer "B.Cu") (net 15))
 (segment (start 86.45 73.09) (end 85 74.54) (width 0.5) (layer "F.Cu") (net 5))
 (segment (start 87 76.54) (end 85 74.54) (width 0.5) (layer "F.Cu") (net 5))
 (segment (start 118.5 85) (end 107.5 96) (width 0.5) (layer "F.Cu") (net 5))
 (segment (start 118.5 64.62) (end 118.5 85) (width 0.5) (layer "F.Cu") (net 5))
 (segment (start 84.66 50.15) (end 86.45 51.94) (width 0.5) (layer "F.Cu") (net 5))
 (segment (start 86.45 51.94) (end 86.45 73.09) (width 0.5) (layer "F.Cu") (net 5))
 (segment (start 131 72.12) (end 121 62.12) (width 0.5) (layer "F.Cu") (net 5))
 (segment (start 87 91) (end 87 76.54) (width 0.5) (layer "F.Cu") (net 5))
 (segment (start 131 77.5) (end 131 72.12) (width 0.5) (layer "F.Cu") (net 5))
 (segment (start 92 96) (end 87 91) (width 0.5) (layer "F.Cu") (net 5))
 (segment (start 121 62.12) (end 118.5 64.62) (width 0.5) (layer "F.Cu") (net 5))
 (segment (start 107.5 96) (end 92 96) (width 0.5) (layer "F.Cu") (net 5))
 (segment (start 105.48 74.54) (end 105.76 74.82) (width 0.5) (layer "B.Cu") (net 29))
 (segment (start 97.7 74.54) (end 105.48 74.54) (width 0.5) (layer "B.Cu") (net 29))
 (segment (start 105.48 72) (end 105.76 72.28) (width 0.5) (layer "B.Cu") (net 28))
 (segment (start 97.7 72) (end 105.48 72) (width 0.5) (layer "B.Cu") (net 28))
 (segment (start 77.3 79.62) (end 77 79.92) (width 0.5) (layer "F.Cu") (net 3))
 (segment (start 85 79.62) (end 77.3 79.62) (width 0.5) (layer "F.Cu") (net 3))
 (segment (start 85 77.08) (end 77.3 77.08) (width 0.5) (layer "F.Cu") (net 4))
 (segment (start 77.3 77.08) (end 77 77.38) (width 0.5) (layer "F.Cu") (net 4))
 (segment (start 84.66 85.04) (end 85 84.7) (width 0.5) (layer "F.Cu") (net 1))
 (segment (start 77.04 85.04) (end 84.66 85.04) (width 0.5) (layer "F.Cu") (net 1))
 (segment (start 77 85) (end 77.04 85.04) (width 0.5) (layer "F.Cu") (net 1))
 (segment (start 85 82.16) (end 77.3 82.16) (width 0.5) (layer "F.Cu") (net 2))
 (segment (start 77.3 82.16) (end 77 82.46) (width 0.5) (layer "F.Cu") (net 2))
 (segment (start 84.39 52.42) (end 84.66 52.69) (width 0.5) (layer "F.Cu") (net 11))
 (segment (start 77 52.42) (end 84.39 52.42) (width 0.5) (layer "F.Cu") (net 11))
 (segment (start 84.39 54.96) (end 84.66 55.23) (width 0.5) (layer "F.Cu") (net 12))
 (segment (start 77 54.96) (end 84.39 54.96) (width 0.5) (layer "F.Cu") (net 12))
 (segment (start 77 57.5) (end 84.39 57.5) (width 0.5) (layer "F.Cu") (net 13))
 (segment (start 84.39 57.5) (end 84.66 57.77) (width 0.5) (layer "F.Cu") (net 13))
 (segment (start 84.39 60.04) (end 84.66 60.31) (width 0.5) (layer "F.Cu") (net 14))
 (segment (start 77 60.04) (end 84.39 60.04) (width 0.5) (layer "F.Cu") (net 14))
 (segment (start 100 64) (end 100 52.79) (width 0.5) (layer "B.Cu") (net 22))
 (segment (start 105.76 69.74) (end 105.74 69.74) (width 0.5) (layer "B.Cu") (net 22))
 (segment (start 100 52.79) (end 97.36 50.15) (width 0.5) (layer "B.Cu") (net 22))
 (segment (start 105.74 69.74) (end 100 64) (width 0.5) (layer "B.Cu") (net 22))
 (segment (start 124.16 94.5) (end 112.74 94.5) (width 0.5) (layer "B.Cu") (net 9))
 (segment (start 131 87.66) (end 124.16 94.5) (width 0.5) (layer "B.Cu") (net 9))
 (segment (start 105.76 87.52) (end 106.02 87.52) (width 0.5) (layer "B.Cu") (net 9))
 (segment (start 112.74 94.5) (end 105.76 87.52) (width 0.5) (layer "B.Cu") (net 9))
 (segment (start 130.86 90.06) (end 121 90.06) (width 0.5) (layer "F.Cu") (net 10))
 (segment (start 131 90.2) (end 130.86 90.06) (width 0.5) (layer "F.Cu") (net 10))
 (segment (start 107.027208 90.06) (end 105.76 90.06) (width 0.5) (layer "B.Cu") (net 8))
 (segment (start 132.5 90.821321) (end 127.921321 95.4) (width 0.5) (layer "B.Cu") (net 8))
 (segment (start 132.5 86.62) (end 132.5 90.821321) (width 0.5) (layer "B.Cu") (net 8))
 (segment (start 127.921321 95.4) (end 112.367208 95.4) (width 0.5) (layer "B.Cu") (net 8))
 (segment (start 112.367208 95.4) (end 107.027208 90.06) (width 0.5) (layer "B.Cu") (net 8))
 (segment (start 131 85.12) (end 132.5 86.62) (width 0.5) (layer "B.Cu") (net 8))
 (segment (start 131 82.58) (end 121.58 92) (width 0.5) (layer "B.Cu") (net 7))
 (segment (start 121.58 92) (end 113 92) (width 0.5) (layer "B.Cu") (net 7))
 (segment (start 105.98 84.98) (end 105.76 84.98) (width 0.5) (layer "B.Cu") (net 7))
 (segment (start 113 92) (end 105.98 84.98) (width 0.5) (layer "B.Cu") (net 7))
 (segment (start 100.9 51.15) (end 100.9 62.34) (width 0.5) (layer "B.Cu") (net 23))
 (segment (start 97.36 47.61) (end 100.9 51.15) (width 0.5) (layer "B.Cu") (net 23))
 (segment (start 100.9 62.34) (end 105.76 67.2) (width 0.5) (layer "B.Cu") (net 23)))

